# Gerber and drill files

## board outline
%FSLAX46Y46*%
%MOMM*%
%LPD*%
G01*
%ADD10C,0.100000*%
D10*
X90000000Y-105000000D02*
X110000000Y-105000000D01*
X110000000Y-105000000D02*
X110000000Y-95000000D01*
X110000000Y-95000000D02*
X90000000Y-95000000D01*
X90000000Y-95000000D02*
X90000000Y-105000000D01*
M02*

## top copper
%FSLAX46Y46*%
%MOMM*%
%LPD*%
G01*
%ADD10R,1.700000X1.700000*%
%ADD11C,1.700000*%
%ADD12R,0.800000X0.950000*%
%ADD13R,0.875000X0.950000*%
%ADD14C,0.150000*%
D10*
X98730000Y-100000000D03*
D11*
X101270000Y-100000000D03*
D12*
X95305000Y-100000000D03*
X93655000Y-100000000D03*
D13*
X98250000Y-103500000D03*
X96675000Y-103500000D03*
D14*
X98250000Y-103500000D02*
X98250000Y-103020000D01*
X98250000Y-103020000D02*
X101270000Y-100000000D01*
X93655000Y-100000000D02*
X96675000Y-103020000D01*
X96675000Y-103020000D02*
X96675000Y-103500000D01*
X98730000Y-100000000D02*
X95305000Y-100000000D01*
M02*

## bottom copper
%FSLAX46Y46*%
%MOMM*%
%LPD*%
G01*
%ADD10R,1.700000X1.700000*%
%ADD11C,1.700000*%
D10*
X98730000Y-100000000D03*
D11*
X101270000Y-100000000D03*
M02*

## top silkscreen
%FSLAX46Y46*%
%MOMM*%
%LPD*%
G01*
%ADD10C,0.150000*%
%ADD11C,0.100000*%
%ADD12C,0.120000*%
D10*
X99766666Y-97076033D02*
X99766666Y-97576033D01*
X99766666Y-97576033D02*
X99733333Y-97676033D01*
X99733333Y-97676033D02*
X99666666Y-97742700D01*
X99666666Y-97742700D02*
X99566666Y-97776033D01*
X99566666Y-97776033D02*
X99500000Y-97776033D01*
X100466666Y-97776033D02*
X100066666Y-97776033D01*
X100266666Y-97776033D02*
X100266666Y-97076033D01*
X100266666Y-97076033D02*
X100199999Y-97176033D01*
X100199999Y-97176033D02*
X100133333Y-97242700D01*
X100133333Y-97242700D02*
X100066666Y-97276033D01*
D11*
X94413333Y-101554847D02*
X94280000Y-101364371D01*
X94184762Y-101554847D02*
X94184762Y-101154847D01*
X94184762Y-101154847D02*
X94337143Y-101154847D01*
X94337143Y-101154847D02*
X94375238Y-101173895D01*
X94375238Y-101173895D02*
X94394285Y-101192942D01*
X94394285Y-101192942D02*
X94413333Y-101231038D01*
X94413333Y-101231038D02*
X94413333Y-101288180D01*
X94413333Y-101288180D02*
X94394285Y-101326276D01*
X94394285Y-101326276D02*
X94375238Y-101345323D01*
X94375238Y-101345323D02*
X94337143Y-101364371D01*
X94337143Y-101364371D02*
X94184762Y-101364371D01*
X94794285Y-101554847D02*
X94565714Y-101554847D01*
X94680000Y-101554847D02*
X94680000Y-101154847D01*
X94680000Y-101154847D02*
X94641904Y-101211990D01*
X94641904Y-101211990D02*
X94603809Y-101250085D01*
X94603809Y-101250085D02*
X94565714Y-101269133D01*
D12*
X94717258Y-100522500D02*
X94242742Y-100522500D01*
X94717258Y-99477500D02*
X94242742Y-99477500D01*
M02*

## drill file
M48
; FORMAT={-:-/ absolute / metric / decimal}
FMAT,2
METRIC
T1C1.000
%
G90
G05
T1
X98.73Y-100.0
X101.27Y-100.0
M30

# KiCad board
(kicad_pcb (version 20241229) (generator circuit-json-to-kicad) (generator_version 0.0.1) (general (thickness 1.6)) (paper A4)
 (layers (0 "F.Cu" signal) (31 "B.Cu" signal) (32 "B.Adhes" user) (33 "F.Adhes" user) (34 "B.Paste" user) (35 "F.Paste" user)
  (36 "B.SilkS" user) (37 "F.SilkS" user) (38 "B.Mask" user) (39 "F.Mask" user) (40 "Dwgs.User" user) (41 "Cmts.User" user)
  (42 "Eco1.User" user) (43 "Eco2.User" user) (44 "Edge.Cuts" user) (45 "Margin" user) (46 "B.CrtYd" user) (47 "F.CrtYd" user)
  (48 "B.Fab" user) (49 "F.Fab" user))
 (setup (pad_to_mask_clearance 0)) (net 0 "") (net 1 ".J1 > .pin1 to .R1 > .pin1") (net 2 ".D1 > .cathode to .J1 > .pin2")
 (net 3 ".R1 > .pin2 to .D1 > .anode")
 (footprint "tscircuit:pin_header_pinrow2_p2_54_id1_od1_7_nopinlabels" (layer F.Cu) (at 100 100 0)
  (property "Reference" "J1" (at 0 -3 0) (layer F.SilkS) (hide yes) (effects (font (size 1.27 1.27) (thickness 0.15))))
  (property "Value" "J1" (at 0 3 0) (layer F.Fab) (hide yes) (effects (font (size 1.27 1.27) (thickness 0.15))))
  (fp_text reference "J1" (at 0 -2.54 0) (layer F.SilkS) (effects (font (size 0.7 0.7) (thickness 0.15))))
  (pad "1" thru_hole rect (at -1.27 0 0) (size 1.7 1.7) (drill 1) (layers *.Cu *.Mask) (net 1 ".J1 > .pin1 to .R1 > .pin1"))
  (pad "2" thru_hole circle (at 1.27 0 0) (size 1.7 1.7) (drill 1) (layers *.Cu *.Mask) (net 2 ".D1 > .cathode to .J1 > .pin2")))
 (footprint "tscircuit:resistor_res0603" (layer F.Cu) (at 94.48 100 180)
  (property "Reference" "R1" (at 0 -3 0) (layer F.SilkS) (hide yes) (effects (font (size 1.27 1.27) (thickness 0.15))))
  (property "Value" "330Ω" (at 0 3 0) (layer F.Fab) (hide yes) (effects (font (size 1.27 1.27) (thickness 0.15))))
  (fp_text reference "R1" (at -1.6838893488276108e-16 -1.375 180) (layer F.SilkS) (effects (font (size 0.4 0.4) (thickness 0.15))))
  (fp_line (start -0.2372579999999998 -0.5225) (end 0.2372579999999997 -0.5225) (stroke (width 0.12) (type default)) (layer F.SilkS))
  (fp_line (start -0.2372579999999997 0.5225) (end 0.2372579999999998 0.5225) (stroke (width 0.12) (type default)) (layer F.SilkS))
  (pad "1" smd rect (at -0.8250000000000002 0 0) (size 0.8 0.95) (layers F.Cu F.Mask) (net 1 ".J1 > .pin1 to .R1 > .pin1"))
  (pad "2" smd rect (at 0.8250000000000002 0 0) (size 0.8 0.95) (layers F.Cu F.Mask) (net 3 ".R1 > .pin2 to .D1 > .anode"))
  (pad "" smd rect (at -0.8250000000000002 0 0) (size 0.5599999999999999 0.6649999999999999) (layers F.Paste))
  (pad "" smd rect (at 0.8250000000000002 0 0) (size 0.5599999999999999 0.6649999999999999) (layers F.Paste)))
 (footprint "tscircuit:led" (layer F.Cu) (at 97.4625 103.5 180)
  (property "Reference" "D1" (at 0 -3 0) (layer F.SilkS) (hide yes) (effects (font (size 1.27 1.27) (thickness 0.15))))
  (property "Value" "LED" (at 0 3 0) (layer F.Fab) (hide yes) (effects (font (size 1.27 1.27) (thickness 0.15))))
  (pad "2" smd rect (at -0.7875000000000001 4.440892098500626e-16 0) (size 0.875 0.95) (layers F.Cu F.Mask)
   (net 2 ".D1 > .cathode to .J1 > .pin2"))
  (pad "1" smd rect (at 0.7875000000000001 0 0) (size 0.875 0.95) (layers F.Cu F.Mask) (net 3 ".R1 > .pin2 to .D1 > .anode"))
  (pad "" smd rect (at -0.7875000000000001 4.440892098500626e-16 0) (size 0.6124999999999999 0.6649999999999999) (layers F.Paste))
  (pad "" smd rect (at 0.7875000000000001 0 0) (size 0.6124999999999999 0.6649999999999999) (layers F.Paste)))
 (segment (start 98.25 103.5) (end 98.25 103.02) (width 0.15) (layer F.Cu) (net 2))
 (segment (start 98.25 103.02) (end 101.27 100) (width 0.15) (layer F.Cu) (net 2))
 (segment (start 93.655 100) (end 96.675 103.02) (width 0.15) (layer F.Cu) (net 3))
 (segment (start 96.675 103.02) (end 96.675 103.5) (width 0.15) (layer F.Cu) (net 3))
 (segment (start 98.73 100) (end 95.305 100) (width 0.15) (layer F.Cu) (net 1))
 (gr_line (start 90 105) (end 110 105) (width 0.1) (layer Edge.Cuts))
 (gr_line (start 110 105) (end 110 95) (width 0.1) (layer Edge.Cuts))
 (gr_line (start 110 95) (end 90 95) (width 0.1) (layer Edge.Cuts))
 (gr_line (start 90 95) (end 90 105) (width 0.1) (layer Edge.Cuts)))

